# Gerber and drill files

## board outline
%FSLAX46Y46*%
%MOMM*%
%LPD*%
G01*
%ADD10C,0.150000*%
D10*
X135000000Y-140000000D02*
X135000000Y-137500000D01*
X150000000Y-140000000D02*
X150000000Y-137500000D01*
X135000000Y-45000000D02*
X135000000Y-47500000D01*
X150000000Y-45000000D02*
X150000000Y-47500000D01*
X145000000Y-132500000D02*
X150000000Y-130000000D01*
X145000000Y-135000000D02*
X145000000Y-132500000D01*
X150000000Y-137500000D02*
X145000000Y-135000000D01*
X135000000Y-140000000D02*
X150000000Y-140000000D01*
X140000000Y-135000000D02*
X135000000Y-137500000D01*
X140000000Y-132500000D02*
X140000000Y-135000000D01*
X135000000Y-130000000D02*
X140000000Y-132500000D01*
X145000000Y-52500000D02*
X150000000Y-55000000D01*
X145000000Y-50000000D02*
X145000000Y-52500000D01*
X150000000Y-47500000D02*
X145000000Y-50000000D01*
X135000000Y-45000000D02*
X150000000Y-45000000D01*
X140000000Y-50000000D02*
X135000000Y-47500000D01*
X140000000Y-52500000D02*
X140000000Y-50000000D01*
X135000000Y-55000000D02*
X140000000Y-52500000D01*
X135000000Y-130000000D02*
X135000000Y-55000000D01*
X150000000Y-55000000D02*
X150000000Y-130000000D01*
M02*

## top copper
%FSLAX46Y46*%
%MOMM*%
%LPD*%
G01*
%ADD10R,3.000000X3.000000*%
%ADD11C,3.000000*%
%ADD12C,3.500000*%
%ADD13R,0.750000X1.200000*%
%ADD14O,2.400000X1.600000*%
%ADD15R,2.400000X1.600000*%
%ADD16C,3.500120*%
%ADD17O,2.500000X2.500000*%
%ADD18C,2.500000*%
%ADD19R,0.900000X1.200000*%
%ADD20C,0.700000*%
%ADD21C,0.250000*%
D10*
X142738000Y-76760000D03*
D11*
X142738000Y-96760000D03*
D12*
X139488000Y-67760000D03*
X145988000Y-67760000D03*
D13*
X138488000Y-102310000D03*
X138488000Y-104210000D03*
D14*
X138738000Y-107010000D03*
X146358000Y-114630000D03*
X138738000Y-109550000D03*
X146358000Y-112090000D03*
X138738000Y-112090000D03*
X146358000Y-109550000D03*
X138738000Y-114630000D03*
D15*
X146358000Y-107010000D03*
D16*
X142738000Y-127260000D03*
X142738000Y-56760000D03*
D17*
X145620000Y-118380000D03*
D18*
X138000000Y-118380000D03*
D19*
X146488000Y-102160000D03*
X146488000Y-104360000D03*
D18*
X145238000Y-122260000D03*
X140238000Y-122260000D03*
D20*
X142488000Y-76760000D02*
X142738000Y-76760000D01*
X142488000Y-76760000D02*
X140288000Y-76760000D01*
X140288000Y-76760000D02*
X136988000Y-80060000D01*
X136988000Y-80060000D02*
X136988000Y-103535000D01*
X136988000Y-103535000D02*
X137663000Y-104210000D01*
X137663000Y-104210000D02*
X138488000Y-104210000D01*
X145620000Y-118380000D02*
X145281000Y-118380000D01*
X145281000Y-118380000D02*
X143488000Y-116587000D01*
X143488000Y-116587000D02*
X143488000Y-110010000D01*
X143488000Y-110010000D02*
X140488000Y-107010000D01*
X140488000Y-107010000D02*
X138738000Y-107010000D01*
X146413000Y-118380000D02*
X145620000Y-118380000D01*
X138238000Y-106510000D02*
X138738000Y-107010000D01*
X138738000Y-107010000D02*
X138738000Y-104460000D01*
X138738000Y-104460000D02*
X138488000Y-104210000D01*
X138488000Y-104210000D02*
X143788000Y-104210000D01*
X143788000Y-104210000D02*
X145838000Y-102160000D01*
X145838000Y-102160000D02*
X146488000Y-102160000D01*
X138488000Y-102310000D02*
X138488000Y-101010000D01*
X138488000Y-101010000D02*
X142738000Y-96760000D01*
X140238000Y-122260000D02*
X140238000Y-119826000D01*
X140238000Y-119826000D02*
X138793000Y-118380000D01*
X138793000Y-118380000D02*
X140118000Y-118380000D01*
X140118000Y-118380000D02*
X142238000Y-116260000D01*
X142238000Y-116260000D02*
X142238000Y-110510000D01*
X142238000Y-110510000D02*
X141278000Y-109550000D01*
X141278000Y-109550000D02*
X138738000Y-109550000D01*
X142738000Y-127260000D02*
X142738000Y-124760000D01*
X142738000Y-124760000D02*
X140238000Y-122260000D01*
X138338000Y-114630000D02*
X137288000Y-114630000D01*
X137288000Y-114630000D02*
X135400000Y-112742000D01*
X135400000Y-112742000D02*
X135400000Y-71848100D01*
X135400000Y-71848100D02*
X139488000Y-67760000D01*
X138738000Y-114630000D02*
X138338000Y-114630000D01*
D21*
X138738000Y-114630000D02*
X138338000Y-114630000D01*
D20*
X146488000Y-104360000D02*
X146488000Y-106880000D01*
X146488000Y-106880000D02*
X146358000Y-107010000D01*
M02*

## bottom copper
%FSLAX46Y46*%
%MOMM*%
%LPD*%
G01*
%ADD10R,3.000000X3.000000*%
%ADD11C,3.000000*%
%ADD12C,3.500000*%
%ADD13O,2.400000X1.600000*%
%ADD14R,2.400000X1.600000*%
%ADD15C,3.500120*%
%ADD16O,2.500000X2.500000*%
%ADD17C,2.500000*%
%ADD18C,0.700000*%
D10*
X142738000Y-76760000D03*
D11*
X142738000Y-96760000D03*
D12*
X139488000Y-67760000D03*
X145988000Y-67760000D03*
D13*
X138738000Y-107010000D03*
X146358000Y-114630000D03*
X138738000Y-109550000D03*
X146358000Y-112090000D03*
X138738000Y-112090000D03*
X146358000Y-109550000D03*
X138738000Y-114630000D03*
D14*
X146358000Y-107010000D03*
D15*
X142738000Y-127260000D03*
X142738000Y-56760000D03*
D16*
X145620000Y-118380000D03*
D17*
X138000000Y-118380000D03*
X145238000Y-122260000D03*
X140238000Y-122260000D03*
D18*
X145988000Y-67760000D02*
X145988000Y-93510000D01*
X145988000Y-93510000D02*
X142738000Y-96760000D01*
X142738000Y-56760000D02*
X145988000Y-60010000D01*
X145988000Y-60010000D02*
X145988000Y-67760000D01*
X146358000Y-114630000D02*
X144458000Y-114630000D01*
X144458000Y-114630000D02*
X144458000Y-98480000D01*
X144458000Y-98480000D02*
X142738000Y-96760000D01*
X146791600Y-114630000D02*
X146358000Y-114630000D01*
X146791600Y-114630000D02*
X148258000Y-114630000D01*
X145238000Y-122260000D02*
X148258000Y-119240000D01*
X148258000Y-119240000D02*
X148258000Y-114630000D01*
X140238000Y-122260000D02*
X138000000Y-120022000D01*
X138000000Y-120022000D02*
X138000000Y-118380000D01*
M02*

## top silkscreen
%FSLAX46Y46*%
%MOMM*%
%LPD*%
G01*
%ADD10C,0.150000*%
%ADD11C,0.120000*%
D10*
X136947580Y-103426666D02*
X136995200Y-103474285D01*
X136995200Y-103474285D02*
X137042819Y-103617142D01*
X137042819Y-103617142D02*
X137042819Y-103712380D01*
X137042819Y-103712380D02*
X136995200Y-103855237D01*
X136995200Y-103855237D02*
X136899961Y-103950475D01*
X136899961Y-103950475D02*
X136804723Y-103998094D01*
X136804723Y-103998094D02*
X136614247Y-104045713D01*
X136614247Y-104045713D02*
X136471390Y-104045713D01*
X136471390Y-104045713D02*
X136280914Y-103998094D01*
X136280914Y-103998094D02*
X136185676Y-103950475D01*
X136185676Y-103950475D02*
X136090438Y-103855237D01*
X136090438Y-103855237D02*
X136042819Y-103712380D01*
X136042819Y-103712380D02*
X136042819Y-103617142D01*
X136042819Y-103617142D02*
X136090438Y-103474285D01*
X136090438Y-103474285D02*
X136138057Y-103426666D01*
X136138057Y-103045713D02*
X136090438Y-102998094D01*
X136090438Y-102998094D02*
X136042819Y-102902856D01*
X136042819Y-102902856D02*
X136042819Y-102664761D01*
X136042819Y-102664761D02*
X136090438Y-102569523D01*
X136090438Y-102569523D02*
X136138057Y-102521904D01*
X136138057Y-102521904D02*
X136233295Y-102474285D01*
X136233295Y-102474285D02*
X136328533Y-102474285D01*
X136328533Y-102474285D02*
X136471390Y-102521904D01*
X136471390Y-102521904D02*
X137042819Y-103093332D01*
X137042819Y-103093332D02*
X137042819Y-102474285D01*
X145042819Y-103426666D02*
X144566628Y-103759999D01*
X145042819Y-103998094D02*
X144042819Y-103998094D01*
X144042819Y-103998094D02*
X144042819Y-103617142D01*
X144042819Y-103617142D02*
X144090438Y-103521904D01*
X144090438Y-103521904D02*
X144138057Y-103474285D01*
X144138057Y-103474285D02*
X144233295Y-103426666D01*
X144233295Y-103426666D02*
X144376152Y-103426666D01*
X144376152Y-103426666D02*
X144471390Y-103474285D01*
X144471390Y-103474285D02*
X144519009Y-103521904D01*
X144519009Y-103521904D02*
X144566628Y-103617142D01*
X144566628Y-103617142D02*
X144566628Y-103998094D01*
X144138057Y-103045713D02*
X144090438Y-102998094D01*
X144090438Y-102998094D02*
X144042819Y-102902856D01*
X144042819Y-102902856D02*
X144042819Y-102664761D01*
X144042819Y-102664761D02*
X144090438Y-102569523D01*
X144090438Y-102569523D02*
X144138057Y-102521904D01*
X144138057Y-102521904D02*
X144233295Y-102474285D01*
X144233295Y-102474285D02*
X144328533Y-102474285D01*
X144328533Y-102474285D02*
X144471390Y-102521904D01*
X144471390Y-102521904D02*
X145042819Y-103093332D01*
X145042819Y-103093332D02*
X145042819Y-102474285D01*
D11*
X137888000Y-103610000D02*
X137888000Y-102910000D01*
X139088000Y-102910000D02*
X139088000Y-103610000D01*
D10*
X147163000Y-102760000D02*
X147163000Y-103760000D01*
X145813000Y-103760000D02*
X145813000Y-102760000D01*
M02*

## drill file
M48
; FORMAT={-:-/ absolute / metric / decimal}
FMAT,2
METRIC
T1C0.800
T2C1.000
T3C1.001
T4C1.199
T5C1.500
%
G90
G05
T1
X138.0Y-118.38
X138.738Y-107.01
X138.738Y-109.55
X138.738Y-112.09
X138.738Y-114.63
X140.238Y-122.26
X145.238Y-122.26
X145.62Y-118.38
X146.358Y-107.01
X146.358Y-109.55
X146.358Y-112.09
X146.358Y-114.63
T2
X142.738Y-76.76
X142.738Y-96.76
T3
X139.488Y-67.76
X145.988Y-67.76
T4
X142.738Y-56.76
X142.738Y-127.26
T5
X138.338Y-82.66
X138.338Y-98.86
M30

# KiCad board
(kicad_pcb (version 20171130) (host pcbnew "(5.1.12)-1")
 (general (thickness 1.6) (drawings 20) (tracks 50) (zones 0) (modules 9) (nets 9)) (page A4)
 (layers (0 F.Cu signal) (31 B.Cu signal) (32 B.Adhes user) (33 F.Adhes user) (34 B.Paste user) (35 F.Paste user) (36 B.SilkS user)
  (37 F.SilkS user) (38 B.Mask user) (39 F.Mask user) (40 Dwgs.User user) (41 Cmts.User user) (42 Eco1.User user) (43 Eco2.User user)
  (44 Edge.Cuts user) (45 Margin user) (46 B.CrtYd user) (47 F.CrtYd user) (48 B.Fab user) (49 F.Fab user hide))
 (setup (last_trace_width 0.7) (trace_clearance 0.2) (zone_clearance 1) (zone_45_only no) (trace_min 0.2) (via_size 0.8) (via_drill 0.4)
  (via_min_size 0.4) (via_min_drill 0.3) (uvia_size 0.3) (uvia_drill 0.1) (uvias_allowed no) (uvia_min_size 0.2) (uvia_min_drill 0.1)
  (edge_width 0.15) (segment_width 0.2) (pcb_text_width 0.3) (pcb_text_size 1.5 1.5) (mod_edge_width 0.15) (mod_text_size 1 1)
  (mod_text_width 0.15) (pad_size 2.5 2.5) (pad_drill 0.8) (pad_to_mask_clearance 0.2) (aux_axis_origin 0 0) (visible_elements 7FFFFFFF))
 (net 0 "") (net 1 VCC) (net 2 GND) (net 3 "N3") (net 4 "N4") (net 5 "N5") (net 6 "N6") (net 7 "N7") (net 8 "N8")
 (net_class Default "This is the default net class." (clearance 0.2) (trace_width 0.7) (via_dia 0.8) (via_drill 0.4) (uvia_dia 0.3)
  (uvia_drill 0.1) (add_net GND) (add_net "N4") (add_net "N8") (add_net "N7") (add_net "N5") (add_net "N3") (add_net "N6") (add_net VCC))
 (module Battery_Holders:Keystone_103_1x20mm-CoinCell (layer B.Cu) (at 142.738 90.76 270)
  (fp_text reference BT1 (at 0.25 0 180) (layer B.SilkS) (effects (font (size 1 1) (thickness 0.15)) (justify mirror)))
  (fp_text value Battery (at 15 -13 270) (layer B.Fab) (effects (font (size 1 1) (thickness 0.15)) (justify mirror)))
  (pad 1 thru_hole rect (at -14 0 270) (size 3 3) (drill 1) (layers *.Cu *.Mask) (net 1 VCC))
  (pad 2 thru_hole circle (at 6 0 270) (size 3 3) (drill 1) (layers *.Cu *.Mask) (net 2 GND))
  (pad "" np_thru_hole circle (at -8.1 4.4 270) (size 1.5 1.5) (drill 1.5) (layers *.Cu *.Mask))
  (pad "" np_thru_hole circle (at 8.1 4.4 270) (size 1.5 1.5) (drill 1.5) (layers *.Cu *.Mask)))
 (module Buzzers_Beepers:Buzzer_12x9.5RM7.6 (layer B.Cu) (at 142.738 67.76 180)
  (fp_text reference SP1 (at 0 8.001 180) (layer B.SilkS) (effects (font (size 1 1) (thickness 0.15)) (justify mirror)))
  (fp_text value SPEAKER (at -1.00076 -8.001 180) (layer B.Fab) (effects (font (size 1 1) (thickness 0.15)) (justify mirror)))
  (pad 2 thru_hole circle (at 3.25 0 180) (size 3.5 3.5) (drill 1.00076) (layers *.Cu *.Mask) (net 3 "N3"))
  (pad 1 thru_hole circle (at -3.25 0 180) (size 3.5 3.5) (drill 1.00076) (layers *.Cu *.Mask) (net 2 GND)))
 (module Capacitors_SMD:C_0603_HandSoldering (layer F.Cu) (at 138.488 103.26 90)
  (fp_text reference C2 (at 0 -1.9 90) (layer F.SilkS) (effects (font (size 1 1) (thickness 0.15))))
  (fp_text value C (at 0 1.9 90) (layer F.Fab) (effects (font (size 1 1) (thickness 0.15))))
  (fp_line (start -0.35 -0.6) (end 0.35 -0.6) (layer F.SilkS) (width 0.12))
  (fp_line (start 0.35 0.6) (end -0.35 0.6) (layer F.SilkS) (width 0.12))
  (pad 2 smd rect (at 0.95 0 90) (size 1.2 0.75) (layers F.Cu F.Paste F.Mask) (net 2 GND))
  (pad 1 smd rect (at -0.95 0 90) (size 1.2 0.75) (layers F.Cu F.Paste F.Mask) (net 1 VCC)))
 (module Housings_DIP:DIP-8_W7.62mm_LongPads (layer B.Cu) (at 146.358 107.01 180)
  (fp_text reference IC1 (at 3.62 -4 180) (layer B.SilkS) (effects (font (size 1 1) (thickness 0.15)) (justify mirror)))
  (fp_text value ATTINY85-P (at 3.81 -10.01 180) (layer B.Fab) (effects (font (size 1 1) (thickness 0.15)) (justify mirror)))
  (pad 8 thru_hole oval (at 7.62 0 180) (size 2.4 1.6) (drill 0.8) (layers *.Cu *.Mask) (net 1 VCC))
  (pad 4 thru_hole oval (at 0 -7.62 180) (size 2.4 1.6) (drill 0.8) (layers *.Cu *.Mask) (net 2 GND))
  (pad 7 thru_hole oval (at 7.62 -2.54 180) (size 2.4 1.6) (drill 0.8) (layers *.Cu *.Mask) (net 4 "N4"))
  (pad 3 thru_hole oval (at 0 -5.08 180) (size 2.4 1.6) (drill 0.8) (layers *.Cu *.Mask) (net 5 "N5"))
  (pad 6 thru_hole oval (at 7.62 -5.08 180) (size 2.4 1.6) (drill 0.8) (layers *.Cu *.Mask) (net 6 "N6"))
  (pad 2 thru_hole oval (at 0 -2.54 180) (size 2.4 1.6) (drill 0.8) (layers *.Cu *.Mask) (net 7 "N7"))
  (pad 5 thru_hole oval (at 7.62 -7.62 180) (size 2.4 1.6) (drill 0.8) (layers *.Cu *.Mask) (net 3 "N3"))
  (pad 1 thru_hole rect (at 0 0 180) (size 2.4 1.6) (drill 0.8) (layers *.Cu *.Mask) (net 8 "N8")))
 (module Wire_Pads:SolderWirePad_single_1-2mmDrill (layer B.Cu) (at 142.738 127.26 180)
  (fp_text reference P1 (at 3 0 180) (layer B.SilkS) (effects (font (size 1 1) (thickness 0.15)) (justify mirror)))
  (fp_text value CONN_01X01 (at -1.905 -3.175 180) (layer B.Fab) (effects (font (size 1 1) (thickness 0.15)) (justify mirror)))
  (pad 1 thru_hole circle (at 0 0 180) (size 3.50012 3.50012) (drill 1.19888) (layers *.Cu *.Mask) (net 4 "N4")))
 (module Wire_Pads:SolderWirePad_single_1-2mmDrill (layer B.Cu) (at 142.738 56.76 180)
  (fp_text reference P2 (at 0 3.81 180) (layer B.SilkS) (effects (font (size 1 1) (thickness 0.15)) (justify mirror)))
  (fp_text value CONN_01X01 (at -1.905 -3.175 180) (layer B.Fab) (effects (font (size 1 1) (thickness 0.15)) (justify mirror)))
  (pad 1 thru_hole circle (at 0 0 180) (size 3.50012 3.50012) (drill 1.19888) (layers *.Cu *.Mask) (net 2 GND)))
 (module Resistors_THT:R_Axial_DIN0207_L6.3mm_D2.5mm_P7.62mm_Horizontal (layer B.Cu) (at 138 118.38)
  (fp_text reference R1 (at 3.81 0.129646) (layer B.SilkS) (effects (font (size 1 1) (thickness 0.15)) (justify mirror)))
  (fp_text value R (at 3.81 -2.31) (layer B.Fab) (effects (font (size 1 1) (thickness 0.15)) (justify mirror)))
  (pad 2 thru_hole oval (at 7.62 0) (size 2.5 2.5) (drill 0.8) (layers *.Cu *.Mask) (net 1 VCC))
  (pad 1 thru_hole circle (at 0 0) (size 2.5 2.5) (drill 0.8) (layers *.Cu *.Mask) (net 4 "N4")))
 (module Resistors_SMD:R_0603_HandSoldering (layer F.Cu) (at 146.488 103.26 90)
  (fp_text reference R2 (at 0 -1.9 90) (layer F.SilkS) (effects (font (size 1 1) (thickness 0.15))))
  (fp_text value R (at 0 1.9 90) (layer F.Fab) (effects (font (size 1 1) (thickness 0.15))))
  (fp_line (start 0.5 0.675) (end -0.5 0.675) (layer F.SilkS) (width 0.15))
  (fp_line (start -0.5 -0.675) (end 0.5 -0.675) (layer F.SilkS) (width 0.15))
  (pad 2 smd rect (at 1.1 0 90) (size 1.2 0.9) (layers F.Cu F.Paste F.Mask) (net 1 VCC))
  (pad 1 smd rect (at -1.1 0 90) (size 1.2 0.9) (layers F.Cu F.Paste F.Mask) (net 8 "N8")))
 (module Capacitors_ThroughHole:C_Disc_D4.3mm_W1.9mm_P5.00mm (layer B.Cu) (at 140.238 122.26)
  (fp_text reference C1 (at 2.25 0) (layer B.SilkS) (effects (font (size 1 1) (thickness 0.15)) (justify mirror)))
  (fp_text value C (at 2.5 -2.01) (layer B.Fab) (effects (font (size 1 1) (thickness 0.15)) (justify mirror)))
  (pad 2 thru_hole circle (at 5 0) (size 2.5 2.5) (drill 0.8) (layers *.Cu *.Mask) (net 2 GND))
  (pad 1 thru_hole circle (at 0 0) (size 2.5 2.5) (drill 0.8) (layers *.Cu *.Mask) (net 4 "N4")))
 (gr_line (start 135 140) (end 135 137.5) (layer Edge.Cuts) (width 0.15))
 (gr_line (start 150 140) (end 150 137.5) (layer Edge.Cuts) (width 0.15))
 (gr_line (start 135 45) (end 135 47.5) (layer Edge.Cuts) (width 0.15))
 (gr_line (start 150 45) (end 150 47.5) (layer Edge.Cuts) (width 0.15))
 (gr_line (start 145 132.5) (end 150 130) (layer Edge.Cuts) (width 0.15))
 (gr_line (start 145 135) (end 145 132.5) (layer Edge.Cuts) (width 0.15))
 (gr_line (start 150 137.5) (end 145 135) (layer Edge.Cuts) (width 0.15))
 (gr_line (start 135 140) (end 150 140) (layer Edge.Cuts) (width 0.15))
 (gr_line (start 140 135) (end 135 137.5) (layer Edge.Cuts) (width 0.15))
 (gr_line (start 140 132.5) (end 140 135) (layer Edge.Cuts) (width 0.15))
 (gr_line (start 135 130) (end 140 132.5) (layer Edge.Cuts) (width 0.15))
 (gr_line (start 145 52.5) (end 150 55) (layer Edge.Cuts) (width 0.15))
 (gr_line (start 145 50) (end 145 52.5) (layer Edge.Cuts) (width 0.15))
 (gr_line (start 150 47.5) (end 145 50) (layer Edge.Cuts) (width 0.15))
 (gr_line (start 135 45) (end 150 45) (layer Edge.Cuts) (width 0.15))
 (gr_line (start 140 50) (end 135 47.5) (layer Edge.Cuts) (width 0.15))
 (gr_line (start 140 52.5) (end 140 50) (layer Edge.Cuts) (width 0.15))
 (gr_line (start 135 55) (end 140 52.5) (layer Edge.Cuts) (width 0.15))
 (gr_line (start 135 130) (end 135 55) (layer Edge.Cuts) (width 0.15))
 (gr_line (start 150 55) (end 150 130) (layer Edge.Cuts) (width 0.15))
 (segment (start 142.488 76.76) (end 142.738 76.76) (width 0.7) (layer F.Cu) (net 1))
 (segment (start 142.488 76.76) (end 140.288 76.76) (width 0.7) (layer F.Cu) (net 1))
 (segment (start 140.288 76.76) (end 136.988 80.06) (width 0.7) (layer F.Cu) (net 1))
 (segment (start 136.988 80.06) (end 136.988 103.535) (width 0.7) (layer F.Cu) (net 1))
 (segment (start 136.988 103.535) (end 137.663 104.21) (width 0.7) (layer F.Cu) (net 1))
 (segment (start 137.663 104.21) (end 138.488 104.21) (width 0.7) (layer F.Cu) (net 1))
 (segment (start 145.62 118.38) (end 145.281 118.38) (width 0.7) (layer F.Cu) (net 1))
 (segment (start 145.281 118.38) (end 143.488 116.587) (width 0.7) (layer F.Cu) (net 1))
 (segment (start 143.488 116.587) (end 143.488 110.01) (width 0.7) (layer F.Cu) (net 1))
 (segment (start 143.488 110.01) (end 140.488 107.01) (width 0.7) (layer F.Cu) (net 1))
 (segment (start 140.488 107.01) (end 138.738 107.01) (width 0.7) (layer F.Cu) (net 1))
 (segment (start 146.413 118.38) (end 145.62 118.38) (width 0.7) (layer F.Cu) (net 1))
 (segment (start 138.238 106.51) (end 138.738 107.01) (width 0.7) (layer F.Cu) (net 1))
 (segment (start 138.738 107.01) (end 138.738 104.46) (width 0.7) (layer F.Cu) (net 1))
 (segment (start 138.738 104.46) (end 138.488 104.21) (width 0.7) (layer F.Cu) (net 1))
 (segment (start 138.488 104.21) (end 143.788 104.21) (width 0.7) (layer F.Cu) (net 1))
 (segment (start 143.788 104.21) (end 145.838 102.16) (width 0.7) (layer F.Cu) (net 1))
 (segment (start 145.838 102.16) (end 146.488 102.16) (width 0.7) (layer F.Cu) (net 1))
 (segment (start 145.988 67.76) (end 145.988 93.51) (width 0.7) (layer B.Cu) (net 2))
 (segment (start 145.988 93.51) (end 142.738 96.76) (width 0.7) (layer B.Cu) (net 2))
 (segment (start 142.738 56.76) (end 145.988 60.01) (width 0.7) (layer B.Cu) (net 2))
 (segment (start 145.988 60.01) (end 145.988 67.76) (width 0.7) (layer B.Cu) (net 2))
 (segment (start 138.488 102.31) (end 138.488 101.01) (width 0.7) (layer F.Cu) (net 2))
 (segment (start 138.488 101.01) (end 142.738 96.76) (width 0.7) (layer F.Cu) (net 2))
 (segment (start 146.358 114.63) (end 144.458 114.63) (width 0.7) (layer B.Cu) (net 2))
 (segment (start 144.458 114.63) (end 144.458 98.48) (width 0.7) (layer B.Cu) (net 2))
 (segment (start 144.458 98.48) (end 142.738 96.76) (width 0.7) (layer B.Cu) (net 2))
 (segment (start 146.7916 114.63) (end 146.358 114.63) (width 0.7) (layer B.Cu) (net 2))
 (segment (start 146.7916 114.63) (end 148.258 114.63) (width 0.7) (layer B.Cu) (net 2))
 (segment (start 145.238 122.26) (end 148.258 119.24) (width 0.7) (layer B.Cu) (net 2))
 (segment (start 148.258 119.24) (end 148.258 114.63) (width 0.7) (layer B.Cu) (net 2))
 (segment (start 140.238 122.26) (end 138 120.022) (width 0.7) (layer B.Cu) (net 4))
 (segment (start 138 120.022) (end 138 118.38) (width 0.7) (layer B.Cu) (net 4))
 (segment (start 140.238 122.26) (end 140.238 119.826) (width 0.7) (layer F.Cu) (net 4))
 (segment (start 140.238 119.826) (end 138.793 118.38) (width 0.7) (layer F.Cu) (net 4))
 (segment (start 138.793 118.38) (end 140.118 118.38) (width 0.7) (layer F.Cu) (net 4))
 (segment (start 140.118 118.38) (end 142.238 116.26) (width 0.7) (layer F.Cu) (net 4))
 (segment (start 142.238 116.26) (end 142.238 110.51) (width 0.7) (layer F.Cu) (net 4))
 (segment (start 142.238 110.51) (end 141.278 109.55) (width 0.7) (layer F.Cu) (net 4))
 (segment (start 141.278 109.55) (end 138.738 109.55) (width 0.7) (layer F.Cu) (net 4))
 (segment (start 142.738 127.26) (end 142.738 124.76) (width 0.7) (layer F.Cu) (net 4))
 (segment (start 142.738 124.76) (end 140.238 122.26) (width 0.7) (layer F.Cu) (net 4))
 (segment (start 138.338 114.63) (end 137.288 114.63) (width 0.7) (layer F.Cu) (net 3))
 (segment (start 137.288 114.63) (end 135.4 112.742) (width 0.7) (layer F.Cu) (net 3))
 (segment (start 135.4 112.742) (end 135.4 71.8481) (width 0.7) (layer F.Cu) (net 3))
 (segment (start 135.4 71.8481) (end 139.488 67.76) (width 0.7) (layer F.Cu) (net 3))
 (segment (start 138.738 114.63) (end 138.338 114.63) (width 0.7) (layer F.Cu) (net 3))
 (segment (start 138.738 114.63) (end 138.338 114.63) (width 0.25) (layer F.Cu) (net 3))
 (segment (start 146.488 104.36) (end 146.488 106.88) (width 0.7) (layer F.Cu) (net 8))
 (segment (start 146.488 106.88) (end 146.358 107.01) (width 0.7) (layer F.Cu) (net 8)))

